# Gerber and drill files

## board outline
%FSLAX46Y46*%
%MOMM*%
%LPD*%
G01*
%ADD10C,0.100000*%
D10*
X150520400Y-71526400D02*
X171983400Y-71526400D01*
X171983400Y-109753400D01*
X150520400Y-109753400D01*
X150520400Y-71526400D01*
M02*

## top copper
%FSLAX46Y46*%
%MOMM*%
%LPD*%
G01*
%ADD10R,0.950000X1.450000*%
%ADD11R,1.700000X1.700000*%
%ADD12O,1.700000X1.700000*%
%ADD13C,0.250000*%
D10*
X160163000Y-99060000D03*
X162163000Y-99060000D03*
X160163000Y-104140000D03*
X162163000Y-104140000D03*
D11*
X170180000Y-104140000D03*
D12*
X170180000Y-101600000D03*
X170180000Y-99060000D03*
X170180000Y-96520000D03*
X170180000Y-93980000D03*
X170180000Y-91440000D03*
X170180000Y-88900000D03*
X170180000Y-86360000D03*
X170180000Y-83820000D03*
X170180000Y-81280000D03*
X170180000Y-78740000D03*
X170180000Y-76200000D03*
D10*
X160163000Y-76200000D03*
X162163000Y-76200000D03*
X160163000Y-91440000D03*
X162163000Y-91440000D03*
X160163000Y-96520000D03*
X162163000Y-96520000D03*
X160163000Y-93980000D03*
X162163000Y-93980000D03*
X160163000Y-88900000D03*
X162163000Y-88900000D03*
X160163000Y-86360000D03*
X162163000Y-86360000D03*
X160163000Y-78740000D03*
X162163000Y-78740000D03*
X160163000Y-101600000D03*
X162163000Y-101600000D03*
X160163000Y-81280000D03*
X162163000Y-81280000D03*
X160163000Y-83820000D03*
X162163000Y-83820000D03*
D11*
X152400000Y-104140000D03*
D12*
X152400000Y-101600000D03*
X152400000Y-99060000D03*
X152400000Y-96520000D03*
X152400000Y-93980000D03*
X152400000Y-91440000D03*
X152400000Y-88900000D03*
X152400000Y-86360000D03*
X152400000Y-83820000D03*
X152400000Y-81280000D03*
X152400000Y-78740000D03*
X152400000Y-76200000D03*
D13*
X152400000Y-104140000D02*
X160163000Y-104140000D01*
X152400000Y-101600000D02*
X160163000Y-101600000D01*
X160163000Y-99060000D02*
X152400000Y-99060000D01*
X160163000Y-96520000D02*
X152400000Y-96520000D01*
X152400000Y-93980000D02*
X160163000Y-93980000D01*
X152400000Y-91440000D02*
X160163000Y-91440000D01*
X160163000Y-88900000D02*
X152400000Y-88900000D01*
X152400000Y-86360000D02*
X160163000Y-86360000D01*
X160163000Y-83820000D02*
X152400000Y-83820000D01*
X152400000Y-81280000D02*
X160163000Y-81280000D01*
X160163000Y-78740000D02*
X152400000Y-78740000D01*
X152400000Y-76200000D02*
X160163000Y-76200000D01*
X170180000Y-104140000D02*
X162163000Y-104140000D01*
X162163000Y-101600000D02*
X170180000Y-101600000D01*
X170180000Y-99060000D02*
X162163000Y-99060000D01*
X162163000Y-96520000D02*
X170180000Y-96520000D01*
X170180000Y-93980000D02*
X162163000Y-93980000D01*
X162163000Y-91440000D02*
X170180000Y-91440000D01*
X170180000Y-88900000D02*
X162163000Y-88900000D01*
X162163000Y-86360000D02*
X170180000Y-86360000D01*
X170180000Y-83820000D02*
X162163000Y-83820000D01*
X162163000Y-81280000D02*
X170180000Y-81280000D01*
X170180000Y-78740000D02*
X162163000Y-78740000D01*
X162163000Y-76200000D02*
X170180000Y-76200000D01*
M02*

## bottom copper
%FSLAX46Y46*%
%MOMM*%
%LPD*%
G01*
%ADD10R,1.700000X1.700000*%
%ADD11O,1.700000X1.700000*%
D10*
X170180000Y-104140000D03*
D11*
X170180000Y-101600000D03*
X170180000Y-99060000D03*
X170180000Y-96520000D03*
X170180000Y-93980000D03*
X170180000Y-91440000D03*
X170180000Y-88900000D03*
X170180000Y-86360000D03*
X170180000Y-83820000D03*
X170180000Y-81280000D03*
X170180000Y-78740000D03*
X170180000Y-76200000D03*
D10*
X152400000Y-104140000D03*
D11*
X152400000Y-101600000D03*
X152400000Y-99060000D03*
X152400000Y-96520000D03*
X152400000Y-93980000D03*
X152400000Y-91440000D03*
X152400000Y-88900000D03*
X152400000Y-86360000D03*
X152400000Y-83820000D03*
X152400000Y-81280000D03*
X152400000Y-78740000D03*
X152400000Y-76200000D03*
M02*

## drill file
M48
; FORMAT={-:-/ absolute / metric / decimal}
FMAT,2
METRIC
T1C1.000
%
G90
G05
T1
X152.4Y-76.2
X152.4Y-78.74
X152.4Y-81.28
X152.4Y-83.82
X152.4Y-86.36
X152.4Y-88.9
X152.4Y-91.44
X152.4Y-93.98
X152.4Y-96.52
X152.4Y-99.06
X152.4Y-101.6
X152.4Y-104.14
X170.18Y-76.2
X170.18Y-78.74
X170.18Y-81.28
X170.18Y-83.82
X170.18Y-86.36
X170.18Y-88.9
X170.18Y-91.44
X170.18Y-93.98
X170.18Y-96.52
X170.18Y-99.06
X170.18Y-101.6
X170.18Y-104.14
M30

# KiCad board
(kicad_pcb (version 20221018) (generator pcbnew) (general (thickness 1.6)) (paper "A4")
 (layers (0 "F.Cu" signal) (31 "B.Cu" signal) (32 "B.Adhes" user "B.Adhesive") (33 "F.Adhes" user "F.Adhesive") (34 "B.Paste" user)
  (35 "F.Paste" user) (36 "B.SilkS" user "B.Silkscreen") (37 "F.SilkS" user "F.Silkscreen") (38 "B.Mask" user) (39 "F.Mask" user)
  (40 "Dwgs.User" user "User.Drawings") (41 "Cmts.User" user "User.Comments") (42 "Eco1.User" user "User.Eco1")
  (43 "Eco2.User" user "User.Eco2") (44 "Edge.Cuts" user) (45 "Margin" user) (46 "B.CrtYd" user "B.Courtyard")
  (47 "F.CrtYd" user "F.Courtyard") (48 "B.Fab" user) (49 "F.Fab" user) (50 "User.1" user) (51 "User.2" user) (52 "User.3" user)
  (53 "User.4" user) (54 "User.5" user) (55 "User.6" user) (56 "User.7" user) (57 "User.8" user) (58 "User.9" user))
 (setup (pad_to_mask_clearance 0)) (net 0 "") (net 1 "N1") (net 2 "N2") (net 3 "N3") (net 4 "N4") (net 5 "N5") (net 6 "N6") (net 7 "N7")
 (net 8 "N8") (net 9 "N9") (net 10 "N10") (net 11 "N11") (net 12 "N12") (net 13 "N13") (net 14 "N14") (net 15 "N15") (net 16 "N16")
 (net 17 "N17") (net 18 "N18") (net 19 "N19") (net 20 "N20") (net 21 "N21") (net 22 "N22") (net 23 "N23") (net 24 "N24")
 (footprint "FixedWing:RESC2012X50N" (layer "F.Cu") (at 161.163 99.06)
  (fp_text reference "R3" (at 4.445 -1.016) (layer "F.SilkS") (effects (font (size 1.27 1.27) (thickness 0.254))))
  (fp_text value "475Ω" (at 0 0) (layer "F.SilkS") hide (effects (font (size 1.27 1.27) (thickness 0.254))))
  (pad "1" smd rect (at -1 0) (size 0.95 1.45) (layers "F.Cu" "F.Paste" "F.Mask") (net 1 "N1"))
  (pad "2" smd rect (at 1 0) (size 0.95 1.45) (layers "F.Cu" "F.Paste" "F.Mask") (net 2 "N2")))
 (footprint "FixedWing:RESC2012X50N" (layer "F.Cu") (at 161.163 104.14)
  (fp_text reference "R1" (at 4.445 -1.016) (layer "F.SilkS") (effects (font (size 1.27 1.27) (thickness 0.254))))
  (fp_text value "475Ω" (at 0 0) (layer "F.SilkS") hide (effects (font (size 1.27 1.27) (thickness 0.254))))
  (pad "1" smd rect (at -1 0) (size 0.95 1.45) (layers "F.Cu" "F.Paste" "F.Mask") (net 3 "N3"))
  (pad "2" smd rect (at 1 0) (size 0.95 1.45) (layers "F.Cu" "F.Paste" "F.Mask") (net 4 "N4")))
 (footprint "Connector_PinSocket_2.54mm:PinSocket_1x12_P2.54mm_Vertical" (layer "F.Cu") (at 170.18 104.14 180)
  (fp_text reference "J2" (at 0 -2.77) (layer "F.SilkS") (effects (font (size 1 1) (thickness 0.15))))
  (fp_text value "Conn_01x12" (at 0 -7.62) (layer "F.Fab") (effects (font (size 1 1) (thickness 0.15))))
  (pad "1" thru_hole rect (at 0 0 180) (size 1.7 1.7) (drill 1) (layers "*.Cu" "*.Mask") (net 4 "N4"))
  (pad "2" thru_hole oval (at 0 2.54 180) (size 1.7 1.7) (drill 1) (layers "*.Cu" "*.Mask") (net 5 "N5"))
  (pad "3" thru_hole oval (at 0 5.08 180) (size 1.7 1.7) (drill 1) (layers "*.Cu" "*.Mask") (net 2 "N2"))
  (pad "4" thru_hole oval (at 0 7.62 180) (size 1.7 1.7) (drill 1) (layers "*.Cu" "*.Mask") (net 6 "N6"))
  (pad "5" thru_hole oval (at 0 10.16 180) (size 1.7 1.7) (drill 1) (layers "*.Cu" "*.Mask") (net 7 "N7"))
  (pad "6" thru_hole oval (at 0 12.7 180) (size 1.7 1.7) (drill 1) (layers "*.Cu" "*.Mask") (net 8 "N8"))
  (pad "7" thru_hole oval (at 0 15.24 180) (size 1.7 1.7) (drill 1) (layers "*.Cu" "*.Mask") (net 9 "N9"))
  (pad "8" thru_hole oval (at 0 17.78 180) (size 1.7 1.7) (drill 1) (layers "*.Cu" "*.Mask") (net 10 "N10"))
  (pad "9" thru_hole oval (at 0 20.32 180) (size 1.7 1.7) (drill 1) (layers "*.Cu" "*.Mask") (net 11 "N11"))
  (pad "10" thru_hole oval (at 0 22.86 180) (size 1.7 1.7) (drill 1) (layers "*.Cu" "*.Mask") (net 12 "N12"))
  (pad "11" thru_hole oval (at 0 25.4 180) (size 1.7 1.7) (drill 1) (layers "*.Cu" "*.Mask") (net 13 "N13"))
  (pad "12" thru_hole oval (at 0 27.94 180) (size 1.7 1.7) (drill 1) (layers "*.Cu" "*.Mask") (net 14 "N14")))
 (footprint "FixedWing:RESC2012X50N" (layer "F.Cu") (at 161.163 76.2)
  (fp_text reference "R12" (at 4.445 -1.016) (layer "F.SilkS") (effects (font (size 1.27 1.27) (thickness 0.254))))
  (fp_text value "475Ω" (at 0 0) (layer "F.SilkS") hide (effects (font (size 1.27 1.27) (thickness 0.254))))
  (pad "1" smd rect (at -1 0) (size 0.95 1.45) (layers "F.Cu" "F.Paste" "F.Mask") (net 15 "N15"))
  (pad "2" smd rect (at 1 0) (size 0.95 1.45) (layers "F.Cu" "F.Paste" "F.Mask") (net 14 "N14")))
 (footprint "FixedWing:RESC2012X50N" (layer "F.Cu") (at 161.163 91.44)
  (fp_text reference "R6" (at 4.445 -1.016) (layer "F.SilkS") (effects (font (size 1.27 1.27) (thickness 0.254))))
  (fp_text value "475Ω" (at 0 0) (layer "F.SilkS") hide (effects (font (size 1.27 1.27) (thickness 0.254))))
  (pad "1" smd rect (at -1 0) (size 0.95 1.45) (layers "F.Cu" "F.Paste" "F.Mask") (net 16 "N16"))
  (pad "2" smd rect (at 1 0) (size 0.95 1.45) (layers "F.Cu" "F.Paste" "F.Mask") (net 8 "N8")))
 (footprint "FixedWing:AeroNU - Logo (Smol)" (layer "F.Cu") (at 161.355749 109.504388)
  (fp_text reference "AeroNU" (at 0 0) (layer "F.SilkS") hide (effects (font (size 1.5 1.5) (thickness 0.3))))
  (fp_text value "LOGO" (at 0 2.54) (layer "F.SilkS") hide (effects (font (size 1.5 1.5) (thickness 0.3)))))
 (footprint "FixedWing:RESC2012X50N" (layer "F.Cu") (at 161.163 96.52)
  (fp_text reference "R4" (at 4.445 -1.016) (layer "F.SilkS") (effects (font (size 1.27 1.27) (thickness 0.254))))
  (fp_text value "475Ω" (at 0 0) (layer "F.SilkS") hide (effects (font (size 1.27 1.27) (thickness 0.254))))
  (pad "1" smd rect (at -1 0) (size 0.95 1.45) (layers "F.Cu" "F.Paste" "F.Mask") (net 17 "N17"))
  (pad "2" smd rect (at 1 0) (size 0.95 1.45) (layers "F.Cu" "F.Paste" "F.Mask") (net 6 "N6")))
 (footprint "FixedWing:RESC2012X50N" (layer "F.Cu") (at 161.163 93.98)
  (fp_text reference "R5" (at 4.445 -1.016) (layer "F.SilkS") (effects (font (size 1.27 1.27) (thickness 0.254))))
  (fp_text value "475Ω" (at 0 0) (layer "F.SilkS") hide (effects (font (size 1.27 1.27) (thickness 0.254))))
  (pad "1" smd rect (at -1 0) (size 0.95 1.45) (layers "F.Cu" "F.Paste" "F.Mask") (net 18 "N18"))
  (pad "2" smd rect (at 1 0) (size 0.95 1.45) (layers "F.Cu" "F.Paste" "F.Mask") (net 7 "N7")))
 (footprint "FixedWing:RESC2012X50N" (layer "F.Cu") (at 161.163 88.9)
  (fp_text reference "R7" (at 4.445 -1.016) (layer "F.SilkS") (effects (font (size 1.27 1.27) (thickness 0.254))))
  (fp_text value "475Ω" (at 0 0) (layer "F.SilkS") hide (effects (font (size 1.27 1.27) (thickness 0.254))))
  (pad "1" smd rect (at -1 0) (size 0.95 1.45) (layers "F.Cu" "F.Paste" "F.Mask") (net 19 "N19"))
  (pad "2" smd rect (at 1 0) (size 0.95 1.45) (layers "F.Cu" "F.Paste" "F.Mask") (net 9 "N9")))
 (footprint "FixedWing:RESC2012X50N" (layer "F.Cu") (at 161.163 86.36)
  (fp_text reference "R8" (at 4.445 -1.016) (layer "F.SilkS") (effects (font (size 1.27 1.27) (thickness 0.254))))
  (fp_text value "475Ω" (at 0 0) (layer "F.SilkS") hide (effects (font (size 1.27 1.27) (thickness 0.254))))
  (pad "1" smd rect (at -1 0) (size 0.95 1.45) (layers "F.Cu" "F.Paste" "F.Mask") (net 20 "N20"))
  (pad "2" smd rect (at 1 0) (size 0.95 1.45) (layers "F.Cu" "F.Paste" "F.Mask") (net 10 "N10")))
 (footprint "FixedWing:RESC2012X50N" (layer "F.Cu") (at 161.163 78.74)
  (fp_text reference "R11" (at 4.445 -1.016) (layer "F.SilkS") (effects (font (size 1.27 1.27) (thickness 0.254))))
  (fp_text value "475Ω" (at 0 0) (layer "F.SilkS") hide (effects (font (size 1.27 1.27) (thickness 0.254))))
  (pad "1" smd rect (at -1 0) (size 0.95 1.45) (layers "F.Cu" "F.Paste" "F.Mask") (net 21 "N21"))
  (pad "2" smd rect (at 1 0) (size 0.95 1.45) (layers "F.Cu" "F.Paste" "F.Mask") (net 13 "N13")))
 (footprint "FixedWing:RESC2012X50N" (layer "F.Cu") (at 161.163 101.6)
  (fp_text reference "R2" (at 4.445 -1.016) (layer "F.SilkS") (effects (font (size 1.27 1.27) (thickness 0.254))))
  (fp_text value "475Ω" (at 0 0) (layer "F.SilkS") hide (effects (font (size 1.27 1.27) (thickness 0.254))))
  (pad "1" smd rect (at -1 0) (size 0.95 1.45) (layers "F.Cu" "F.Paste" "F.Mask") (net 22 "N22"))
  (pad "2" smd rect (at 1 0) (size 0.95 1.45) (layers "F.Cu" "F.Paste" "F.Mask") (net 5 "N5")))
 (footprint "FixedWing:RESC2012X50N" (layer "F.Cu") (at 161.163 81.28)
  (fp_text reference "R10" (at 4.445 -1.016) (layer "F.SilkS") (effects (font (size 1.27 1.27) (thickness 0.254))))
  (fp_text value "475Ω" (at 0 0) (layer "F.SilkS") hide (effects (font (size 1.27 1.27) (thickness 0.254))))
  (pad "1" smd rect (at -1 0) (size 0.95 1.45) (layers "F.Cu" "F.Paste" "F.Mask") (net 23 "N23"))
  (pad "2" smd rect (at 1 0) (size 0.95 1.45) (layers "F.Cu" "F.Paste" "F.Mask") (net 12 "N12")))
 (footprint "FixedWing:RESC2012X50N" (layer "F.Cu") (at 161.163 83.82)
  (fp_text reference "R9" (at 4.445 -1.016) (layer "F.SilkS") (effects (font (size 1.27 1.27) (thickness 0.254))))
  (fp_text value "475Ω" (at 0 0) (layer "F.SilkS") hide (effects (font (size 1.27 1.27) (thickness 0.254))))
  (pad "1" smd rect (at -1 0) (size 0.95 1.45) (layers "F.Cu" "F.Paste" "F.Mask") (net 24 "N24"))
  (pad "2" smd rect (at 1 0) (size 0.95 1.45) (layers "F.Cu" "F.Paste" "F.Mask") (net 11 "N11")))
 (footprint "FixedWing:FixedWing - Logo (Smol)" (layer "F.Cu") (at 161.250214 73.970419)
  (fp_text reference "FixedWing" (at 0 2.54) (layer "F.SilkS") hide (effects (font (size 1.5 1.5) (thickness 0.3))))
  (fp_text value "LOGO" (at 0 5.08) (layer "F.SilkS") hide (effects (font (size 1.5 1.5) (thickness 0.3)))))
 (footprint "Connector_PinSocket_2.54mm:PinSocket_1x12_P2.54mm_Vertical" (layer "F.Cu") (at 152.4 104.14 180)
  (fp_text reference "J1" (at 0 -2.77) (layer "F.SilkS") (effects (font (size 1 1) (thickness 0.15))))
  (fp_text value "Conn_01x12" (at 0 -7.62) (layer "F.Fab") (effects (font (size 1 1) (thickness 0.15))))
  (pad "1" thru_hole rect (at 0 0 180) (size 1.7 1.7) (drill 1) (layers "*.Cu" "*.Mask") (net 3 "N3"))
  (pad "2" thru_hole oval (at 0 2.54 180) (size 1.7 1.7) (drill 1) (layers "*.Cu" "*.Mask") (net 22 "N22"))
  (pad "3" thru_hole oval (at 0 5.08 180) (size 1.7 1.7) (drill 1) (layers "*.Cu" "*.Mask") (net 1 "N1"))
  (pad "4" thru_hole oval (at 0 7.62 180) (size 1.7 1.7) (drill 1) (layers "*.Cu" "*.Mask") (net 17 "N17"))
  (pad "5" thru_hole oval (at 0 10.16 180) (size 1.7 1.7) (drill 1) (layers "*.Cu" "*.Mask") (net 18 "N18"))
  (pad "6" thru_hole oval (at 0 12.7 180) (size 1.7 1.7) (drill 1) (layers "*.Cu" "*.Mask") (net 16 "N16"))
  (pad "7" thru_hole oval (at 0 15.24 180) (size 1.7 1.7) (drill 1) (layers "*.Cu" "*.Mask") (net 19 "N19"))
  (pad "8" thru_hole oval (at 0 17.78 180) (size 1.7 1.7) (drill 1) (layers "*.Cu" "*.Mask") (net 20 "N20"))
  (pad "9" thru_hole oval (at 0 20.32 180) (size 1.7 1.7) (drill 1) (layers "*.Cu" "*.Mask") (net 24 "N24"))
  (pad "10" thru_hole oval (at 0 22.86 180) (size 1.7 1.7) (drill 1) (layers "*.Cu" "*.Mask") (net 23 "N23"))
  (pad "11" thru_hole oval (at 0 25.4 180) (size 1.7 1.7) (drill 1) (layers "*.Cu" "*.Mask") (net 21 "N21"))
  (pad "12" thru_hole oval (at 0 27.94 180) (size 1.7 1.7) (drill 1) (layers "*.Cu" "*.Mask") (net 15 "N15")))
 (gr_rect (start 150.5204 71.5264) (end 171.9834 109.7534) (stroke (width 0.1) (type default)) (fill none) (layer "Edge.Cuts"))
 (segment (start 152.4 104.14) (end 160.163 104.14) (width 0.25) (layer "F.Cu") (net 3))
 (segment (start 152.4 101.6) (end 160.163 101.6) (width 0.25) (layer "F.Cu") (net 22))
 (segment (start 160.163 99.06) (end 152.4 99.06) (width 0.25) (layer "F.Cu") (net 1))
 (segment (start 160.163 96.52) (end 152.4 96.52) (width 0.25) (layer "F.Cu") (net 17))
 (segment (start 152.4 93.98) (end 160.163 93.98) (width 0.25) (layer "F.Cu") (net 18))
 (segment (start 152.4 91.44) (end 160.163 91.44) (width 0.25) (layer "F.Cu") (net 16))
 (segment (start 160.163 88.9) (end 152.4 88.9) (width 0.25) (layer "F.Cu") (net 19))
 (segment (start 152.4 86.36) (end 160.163 86.36) (width 0.25) (layer "F.Cu") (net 20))
 (segment (start 160.163 83.82) (end 152.4 83.82) (width 0.25) (layer "F.Cu") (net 24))
 (segment (start 152.4 81.28) (end 160.163 81.28) (width 0.25) (layer "F.Cu") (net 23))
 (segment (start 160.163 78.74) (end 152.4 78.74) (width 0.25) (layer "F.Cu") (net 21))
 (segment (start 152.4 76.2) (end 160.163 76.2) (width 0.25) (layer "F.Cu") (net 15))
 (segment (start 170.18 104.14) (end 162.163 104.14) (width 0.25) (layer "F.Cu") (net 4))
 (segment (start 162.163 101.6) (end 170.18 101.6) (width 0.25) (layer "F.Cu") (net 5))
 (segment (start 170.18 99.06) (end 162.163 99.06) (width 0.25) (layer "F.Cu") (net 2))
 (segment (start 162.163 96.52) (end 170.18 96.52) (width 0.25) (layer "F.Cu") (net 6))
 (segment (start 170.18 93.98) (end 162.163 93.98) (width 0.25) (layer "F.Cu") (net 7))
 (segment (start 162.163 91.44) (end 170.18 91.44) (width 0.25) (layer "F.Cu") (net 8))
 (segment (start 170.18 88.9) (end 162.163 88.9) (width 0.25) (layer "F.Cu") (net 9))
 (segment (start 162.163 86.36) (end 170.18 86.36) (width 0.25) (layer "F.Cu") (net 10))
 (segment (start 170.18 83.82) (end 162.163 83.82) (width 0.25) (layer "F.Cu") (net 11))
 (segment (start 162.163 81.28) (end 170.18 81.28) (width 0.25) (layer "F.Cu") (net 12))
 (segment (start 170.18 78.74) (end 162.163 78.74) (width 0.25) (layer "F.Cu") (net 13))
 (segment (start 162.163 76.2) (end 170.18 76.2) (width 0.25) (layer "F.Cu") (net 14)))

